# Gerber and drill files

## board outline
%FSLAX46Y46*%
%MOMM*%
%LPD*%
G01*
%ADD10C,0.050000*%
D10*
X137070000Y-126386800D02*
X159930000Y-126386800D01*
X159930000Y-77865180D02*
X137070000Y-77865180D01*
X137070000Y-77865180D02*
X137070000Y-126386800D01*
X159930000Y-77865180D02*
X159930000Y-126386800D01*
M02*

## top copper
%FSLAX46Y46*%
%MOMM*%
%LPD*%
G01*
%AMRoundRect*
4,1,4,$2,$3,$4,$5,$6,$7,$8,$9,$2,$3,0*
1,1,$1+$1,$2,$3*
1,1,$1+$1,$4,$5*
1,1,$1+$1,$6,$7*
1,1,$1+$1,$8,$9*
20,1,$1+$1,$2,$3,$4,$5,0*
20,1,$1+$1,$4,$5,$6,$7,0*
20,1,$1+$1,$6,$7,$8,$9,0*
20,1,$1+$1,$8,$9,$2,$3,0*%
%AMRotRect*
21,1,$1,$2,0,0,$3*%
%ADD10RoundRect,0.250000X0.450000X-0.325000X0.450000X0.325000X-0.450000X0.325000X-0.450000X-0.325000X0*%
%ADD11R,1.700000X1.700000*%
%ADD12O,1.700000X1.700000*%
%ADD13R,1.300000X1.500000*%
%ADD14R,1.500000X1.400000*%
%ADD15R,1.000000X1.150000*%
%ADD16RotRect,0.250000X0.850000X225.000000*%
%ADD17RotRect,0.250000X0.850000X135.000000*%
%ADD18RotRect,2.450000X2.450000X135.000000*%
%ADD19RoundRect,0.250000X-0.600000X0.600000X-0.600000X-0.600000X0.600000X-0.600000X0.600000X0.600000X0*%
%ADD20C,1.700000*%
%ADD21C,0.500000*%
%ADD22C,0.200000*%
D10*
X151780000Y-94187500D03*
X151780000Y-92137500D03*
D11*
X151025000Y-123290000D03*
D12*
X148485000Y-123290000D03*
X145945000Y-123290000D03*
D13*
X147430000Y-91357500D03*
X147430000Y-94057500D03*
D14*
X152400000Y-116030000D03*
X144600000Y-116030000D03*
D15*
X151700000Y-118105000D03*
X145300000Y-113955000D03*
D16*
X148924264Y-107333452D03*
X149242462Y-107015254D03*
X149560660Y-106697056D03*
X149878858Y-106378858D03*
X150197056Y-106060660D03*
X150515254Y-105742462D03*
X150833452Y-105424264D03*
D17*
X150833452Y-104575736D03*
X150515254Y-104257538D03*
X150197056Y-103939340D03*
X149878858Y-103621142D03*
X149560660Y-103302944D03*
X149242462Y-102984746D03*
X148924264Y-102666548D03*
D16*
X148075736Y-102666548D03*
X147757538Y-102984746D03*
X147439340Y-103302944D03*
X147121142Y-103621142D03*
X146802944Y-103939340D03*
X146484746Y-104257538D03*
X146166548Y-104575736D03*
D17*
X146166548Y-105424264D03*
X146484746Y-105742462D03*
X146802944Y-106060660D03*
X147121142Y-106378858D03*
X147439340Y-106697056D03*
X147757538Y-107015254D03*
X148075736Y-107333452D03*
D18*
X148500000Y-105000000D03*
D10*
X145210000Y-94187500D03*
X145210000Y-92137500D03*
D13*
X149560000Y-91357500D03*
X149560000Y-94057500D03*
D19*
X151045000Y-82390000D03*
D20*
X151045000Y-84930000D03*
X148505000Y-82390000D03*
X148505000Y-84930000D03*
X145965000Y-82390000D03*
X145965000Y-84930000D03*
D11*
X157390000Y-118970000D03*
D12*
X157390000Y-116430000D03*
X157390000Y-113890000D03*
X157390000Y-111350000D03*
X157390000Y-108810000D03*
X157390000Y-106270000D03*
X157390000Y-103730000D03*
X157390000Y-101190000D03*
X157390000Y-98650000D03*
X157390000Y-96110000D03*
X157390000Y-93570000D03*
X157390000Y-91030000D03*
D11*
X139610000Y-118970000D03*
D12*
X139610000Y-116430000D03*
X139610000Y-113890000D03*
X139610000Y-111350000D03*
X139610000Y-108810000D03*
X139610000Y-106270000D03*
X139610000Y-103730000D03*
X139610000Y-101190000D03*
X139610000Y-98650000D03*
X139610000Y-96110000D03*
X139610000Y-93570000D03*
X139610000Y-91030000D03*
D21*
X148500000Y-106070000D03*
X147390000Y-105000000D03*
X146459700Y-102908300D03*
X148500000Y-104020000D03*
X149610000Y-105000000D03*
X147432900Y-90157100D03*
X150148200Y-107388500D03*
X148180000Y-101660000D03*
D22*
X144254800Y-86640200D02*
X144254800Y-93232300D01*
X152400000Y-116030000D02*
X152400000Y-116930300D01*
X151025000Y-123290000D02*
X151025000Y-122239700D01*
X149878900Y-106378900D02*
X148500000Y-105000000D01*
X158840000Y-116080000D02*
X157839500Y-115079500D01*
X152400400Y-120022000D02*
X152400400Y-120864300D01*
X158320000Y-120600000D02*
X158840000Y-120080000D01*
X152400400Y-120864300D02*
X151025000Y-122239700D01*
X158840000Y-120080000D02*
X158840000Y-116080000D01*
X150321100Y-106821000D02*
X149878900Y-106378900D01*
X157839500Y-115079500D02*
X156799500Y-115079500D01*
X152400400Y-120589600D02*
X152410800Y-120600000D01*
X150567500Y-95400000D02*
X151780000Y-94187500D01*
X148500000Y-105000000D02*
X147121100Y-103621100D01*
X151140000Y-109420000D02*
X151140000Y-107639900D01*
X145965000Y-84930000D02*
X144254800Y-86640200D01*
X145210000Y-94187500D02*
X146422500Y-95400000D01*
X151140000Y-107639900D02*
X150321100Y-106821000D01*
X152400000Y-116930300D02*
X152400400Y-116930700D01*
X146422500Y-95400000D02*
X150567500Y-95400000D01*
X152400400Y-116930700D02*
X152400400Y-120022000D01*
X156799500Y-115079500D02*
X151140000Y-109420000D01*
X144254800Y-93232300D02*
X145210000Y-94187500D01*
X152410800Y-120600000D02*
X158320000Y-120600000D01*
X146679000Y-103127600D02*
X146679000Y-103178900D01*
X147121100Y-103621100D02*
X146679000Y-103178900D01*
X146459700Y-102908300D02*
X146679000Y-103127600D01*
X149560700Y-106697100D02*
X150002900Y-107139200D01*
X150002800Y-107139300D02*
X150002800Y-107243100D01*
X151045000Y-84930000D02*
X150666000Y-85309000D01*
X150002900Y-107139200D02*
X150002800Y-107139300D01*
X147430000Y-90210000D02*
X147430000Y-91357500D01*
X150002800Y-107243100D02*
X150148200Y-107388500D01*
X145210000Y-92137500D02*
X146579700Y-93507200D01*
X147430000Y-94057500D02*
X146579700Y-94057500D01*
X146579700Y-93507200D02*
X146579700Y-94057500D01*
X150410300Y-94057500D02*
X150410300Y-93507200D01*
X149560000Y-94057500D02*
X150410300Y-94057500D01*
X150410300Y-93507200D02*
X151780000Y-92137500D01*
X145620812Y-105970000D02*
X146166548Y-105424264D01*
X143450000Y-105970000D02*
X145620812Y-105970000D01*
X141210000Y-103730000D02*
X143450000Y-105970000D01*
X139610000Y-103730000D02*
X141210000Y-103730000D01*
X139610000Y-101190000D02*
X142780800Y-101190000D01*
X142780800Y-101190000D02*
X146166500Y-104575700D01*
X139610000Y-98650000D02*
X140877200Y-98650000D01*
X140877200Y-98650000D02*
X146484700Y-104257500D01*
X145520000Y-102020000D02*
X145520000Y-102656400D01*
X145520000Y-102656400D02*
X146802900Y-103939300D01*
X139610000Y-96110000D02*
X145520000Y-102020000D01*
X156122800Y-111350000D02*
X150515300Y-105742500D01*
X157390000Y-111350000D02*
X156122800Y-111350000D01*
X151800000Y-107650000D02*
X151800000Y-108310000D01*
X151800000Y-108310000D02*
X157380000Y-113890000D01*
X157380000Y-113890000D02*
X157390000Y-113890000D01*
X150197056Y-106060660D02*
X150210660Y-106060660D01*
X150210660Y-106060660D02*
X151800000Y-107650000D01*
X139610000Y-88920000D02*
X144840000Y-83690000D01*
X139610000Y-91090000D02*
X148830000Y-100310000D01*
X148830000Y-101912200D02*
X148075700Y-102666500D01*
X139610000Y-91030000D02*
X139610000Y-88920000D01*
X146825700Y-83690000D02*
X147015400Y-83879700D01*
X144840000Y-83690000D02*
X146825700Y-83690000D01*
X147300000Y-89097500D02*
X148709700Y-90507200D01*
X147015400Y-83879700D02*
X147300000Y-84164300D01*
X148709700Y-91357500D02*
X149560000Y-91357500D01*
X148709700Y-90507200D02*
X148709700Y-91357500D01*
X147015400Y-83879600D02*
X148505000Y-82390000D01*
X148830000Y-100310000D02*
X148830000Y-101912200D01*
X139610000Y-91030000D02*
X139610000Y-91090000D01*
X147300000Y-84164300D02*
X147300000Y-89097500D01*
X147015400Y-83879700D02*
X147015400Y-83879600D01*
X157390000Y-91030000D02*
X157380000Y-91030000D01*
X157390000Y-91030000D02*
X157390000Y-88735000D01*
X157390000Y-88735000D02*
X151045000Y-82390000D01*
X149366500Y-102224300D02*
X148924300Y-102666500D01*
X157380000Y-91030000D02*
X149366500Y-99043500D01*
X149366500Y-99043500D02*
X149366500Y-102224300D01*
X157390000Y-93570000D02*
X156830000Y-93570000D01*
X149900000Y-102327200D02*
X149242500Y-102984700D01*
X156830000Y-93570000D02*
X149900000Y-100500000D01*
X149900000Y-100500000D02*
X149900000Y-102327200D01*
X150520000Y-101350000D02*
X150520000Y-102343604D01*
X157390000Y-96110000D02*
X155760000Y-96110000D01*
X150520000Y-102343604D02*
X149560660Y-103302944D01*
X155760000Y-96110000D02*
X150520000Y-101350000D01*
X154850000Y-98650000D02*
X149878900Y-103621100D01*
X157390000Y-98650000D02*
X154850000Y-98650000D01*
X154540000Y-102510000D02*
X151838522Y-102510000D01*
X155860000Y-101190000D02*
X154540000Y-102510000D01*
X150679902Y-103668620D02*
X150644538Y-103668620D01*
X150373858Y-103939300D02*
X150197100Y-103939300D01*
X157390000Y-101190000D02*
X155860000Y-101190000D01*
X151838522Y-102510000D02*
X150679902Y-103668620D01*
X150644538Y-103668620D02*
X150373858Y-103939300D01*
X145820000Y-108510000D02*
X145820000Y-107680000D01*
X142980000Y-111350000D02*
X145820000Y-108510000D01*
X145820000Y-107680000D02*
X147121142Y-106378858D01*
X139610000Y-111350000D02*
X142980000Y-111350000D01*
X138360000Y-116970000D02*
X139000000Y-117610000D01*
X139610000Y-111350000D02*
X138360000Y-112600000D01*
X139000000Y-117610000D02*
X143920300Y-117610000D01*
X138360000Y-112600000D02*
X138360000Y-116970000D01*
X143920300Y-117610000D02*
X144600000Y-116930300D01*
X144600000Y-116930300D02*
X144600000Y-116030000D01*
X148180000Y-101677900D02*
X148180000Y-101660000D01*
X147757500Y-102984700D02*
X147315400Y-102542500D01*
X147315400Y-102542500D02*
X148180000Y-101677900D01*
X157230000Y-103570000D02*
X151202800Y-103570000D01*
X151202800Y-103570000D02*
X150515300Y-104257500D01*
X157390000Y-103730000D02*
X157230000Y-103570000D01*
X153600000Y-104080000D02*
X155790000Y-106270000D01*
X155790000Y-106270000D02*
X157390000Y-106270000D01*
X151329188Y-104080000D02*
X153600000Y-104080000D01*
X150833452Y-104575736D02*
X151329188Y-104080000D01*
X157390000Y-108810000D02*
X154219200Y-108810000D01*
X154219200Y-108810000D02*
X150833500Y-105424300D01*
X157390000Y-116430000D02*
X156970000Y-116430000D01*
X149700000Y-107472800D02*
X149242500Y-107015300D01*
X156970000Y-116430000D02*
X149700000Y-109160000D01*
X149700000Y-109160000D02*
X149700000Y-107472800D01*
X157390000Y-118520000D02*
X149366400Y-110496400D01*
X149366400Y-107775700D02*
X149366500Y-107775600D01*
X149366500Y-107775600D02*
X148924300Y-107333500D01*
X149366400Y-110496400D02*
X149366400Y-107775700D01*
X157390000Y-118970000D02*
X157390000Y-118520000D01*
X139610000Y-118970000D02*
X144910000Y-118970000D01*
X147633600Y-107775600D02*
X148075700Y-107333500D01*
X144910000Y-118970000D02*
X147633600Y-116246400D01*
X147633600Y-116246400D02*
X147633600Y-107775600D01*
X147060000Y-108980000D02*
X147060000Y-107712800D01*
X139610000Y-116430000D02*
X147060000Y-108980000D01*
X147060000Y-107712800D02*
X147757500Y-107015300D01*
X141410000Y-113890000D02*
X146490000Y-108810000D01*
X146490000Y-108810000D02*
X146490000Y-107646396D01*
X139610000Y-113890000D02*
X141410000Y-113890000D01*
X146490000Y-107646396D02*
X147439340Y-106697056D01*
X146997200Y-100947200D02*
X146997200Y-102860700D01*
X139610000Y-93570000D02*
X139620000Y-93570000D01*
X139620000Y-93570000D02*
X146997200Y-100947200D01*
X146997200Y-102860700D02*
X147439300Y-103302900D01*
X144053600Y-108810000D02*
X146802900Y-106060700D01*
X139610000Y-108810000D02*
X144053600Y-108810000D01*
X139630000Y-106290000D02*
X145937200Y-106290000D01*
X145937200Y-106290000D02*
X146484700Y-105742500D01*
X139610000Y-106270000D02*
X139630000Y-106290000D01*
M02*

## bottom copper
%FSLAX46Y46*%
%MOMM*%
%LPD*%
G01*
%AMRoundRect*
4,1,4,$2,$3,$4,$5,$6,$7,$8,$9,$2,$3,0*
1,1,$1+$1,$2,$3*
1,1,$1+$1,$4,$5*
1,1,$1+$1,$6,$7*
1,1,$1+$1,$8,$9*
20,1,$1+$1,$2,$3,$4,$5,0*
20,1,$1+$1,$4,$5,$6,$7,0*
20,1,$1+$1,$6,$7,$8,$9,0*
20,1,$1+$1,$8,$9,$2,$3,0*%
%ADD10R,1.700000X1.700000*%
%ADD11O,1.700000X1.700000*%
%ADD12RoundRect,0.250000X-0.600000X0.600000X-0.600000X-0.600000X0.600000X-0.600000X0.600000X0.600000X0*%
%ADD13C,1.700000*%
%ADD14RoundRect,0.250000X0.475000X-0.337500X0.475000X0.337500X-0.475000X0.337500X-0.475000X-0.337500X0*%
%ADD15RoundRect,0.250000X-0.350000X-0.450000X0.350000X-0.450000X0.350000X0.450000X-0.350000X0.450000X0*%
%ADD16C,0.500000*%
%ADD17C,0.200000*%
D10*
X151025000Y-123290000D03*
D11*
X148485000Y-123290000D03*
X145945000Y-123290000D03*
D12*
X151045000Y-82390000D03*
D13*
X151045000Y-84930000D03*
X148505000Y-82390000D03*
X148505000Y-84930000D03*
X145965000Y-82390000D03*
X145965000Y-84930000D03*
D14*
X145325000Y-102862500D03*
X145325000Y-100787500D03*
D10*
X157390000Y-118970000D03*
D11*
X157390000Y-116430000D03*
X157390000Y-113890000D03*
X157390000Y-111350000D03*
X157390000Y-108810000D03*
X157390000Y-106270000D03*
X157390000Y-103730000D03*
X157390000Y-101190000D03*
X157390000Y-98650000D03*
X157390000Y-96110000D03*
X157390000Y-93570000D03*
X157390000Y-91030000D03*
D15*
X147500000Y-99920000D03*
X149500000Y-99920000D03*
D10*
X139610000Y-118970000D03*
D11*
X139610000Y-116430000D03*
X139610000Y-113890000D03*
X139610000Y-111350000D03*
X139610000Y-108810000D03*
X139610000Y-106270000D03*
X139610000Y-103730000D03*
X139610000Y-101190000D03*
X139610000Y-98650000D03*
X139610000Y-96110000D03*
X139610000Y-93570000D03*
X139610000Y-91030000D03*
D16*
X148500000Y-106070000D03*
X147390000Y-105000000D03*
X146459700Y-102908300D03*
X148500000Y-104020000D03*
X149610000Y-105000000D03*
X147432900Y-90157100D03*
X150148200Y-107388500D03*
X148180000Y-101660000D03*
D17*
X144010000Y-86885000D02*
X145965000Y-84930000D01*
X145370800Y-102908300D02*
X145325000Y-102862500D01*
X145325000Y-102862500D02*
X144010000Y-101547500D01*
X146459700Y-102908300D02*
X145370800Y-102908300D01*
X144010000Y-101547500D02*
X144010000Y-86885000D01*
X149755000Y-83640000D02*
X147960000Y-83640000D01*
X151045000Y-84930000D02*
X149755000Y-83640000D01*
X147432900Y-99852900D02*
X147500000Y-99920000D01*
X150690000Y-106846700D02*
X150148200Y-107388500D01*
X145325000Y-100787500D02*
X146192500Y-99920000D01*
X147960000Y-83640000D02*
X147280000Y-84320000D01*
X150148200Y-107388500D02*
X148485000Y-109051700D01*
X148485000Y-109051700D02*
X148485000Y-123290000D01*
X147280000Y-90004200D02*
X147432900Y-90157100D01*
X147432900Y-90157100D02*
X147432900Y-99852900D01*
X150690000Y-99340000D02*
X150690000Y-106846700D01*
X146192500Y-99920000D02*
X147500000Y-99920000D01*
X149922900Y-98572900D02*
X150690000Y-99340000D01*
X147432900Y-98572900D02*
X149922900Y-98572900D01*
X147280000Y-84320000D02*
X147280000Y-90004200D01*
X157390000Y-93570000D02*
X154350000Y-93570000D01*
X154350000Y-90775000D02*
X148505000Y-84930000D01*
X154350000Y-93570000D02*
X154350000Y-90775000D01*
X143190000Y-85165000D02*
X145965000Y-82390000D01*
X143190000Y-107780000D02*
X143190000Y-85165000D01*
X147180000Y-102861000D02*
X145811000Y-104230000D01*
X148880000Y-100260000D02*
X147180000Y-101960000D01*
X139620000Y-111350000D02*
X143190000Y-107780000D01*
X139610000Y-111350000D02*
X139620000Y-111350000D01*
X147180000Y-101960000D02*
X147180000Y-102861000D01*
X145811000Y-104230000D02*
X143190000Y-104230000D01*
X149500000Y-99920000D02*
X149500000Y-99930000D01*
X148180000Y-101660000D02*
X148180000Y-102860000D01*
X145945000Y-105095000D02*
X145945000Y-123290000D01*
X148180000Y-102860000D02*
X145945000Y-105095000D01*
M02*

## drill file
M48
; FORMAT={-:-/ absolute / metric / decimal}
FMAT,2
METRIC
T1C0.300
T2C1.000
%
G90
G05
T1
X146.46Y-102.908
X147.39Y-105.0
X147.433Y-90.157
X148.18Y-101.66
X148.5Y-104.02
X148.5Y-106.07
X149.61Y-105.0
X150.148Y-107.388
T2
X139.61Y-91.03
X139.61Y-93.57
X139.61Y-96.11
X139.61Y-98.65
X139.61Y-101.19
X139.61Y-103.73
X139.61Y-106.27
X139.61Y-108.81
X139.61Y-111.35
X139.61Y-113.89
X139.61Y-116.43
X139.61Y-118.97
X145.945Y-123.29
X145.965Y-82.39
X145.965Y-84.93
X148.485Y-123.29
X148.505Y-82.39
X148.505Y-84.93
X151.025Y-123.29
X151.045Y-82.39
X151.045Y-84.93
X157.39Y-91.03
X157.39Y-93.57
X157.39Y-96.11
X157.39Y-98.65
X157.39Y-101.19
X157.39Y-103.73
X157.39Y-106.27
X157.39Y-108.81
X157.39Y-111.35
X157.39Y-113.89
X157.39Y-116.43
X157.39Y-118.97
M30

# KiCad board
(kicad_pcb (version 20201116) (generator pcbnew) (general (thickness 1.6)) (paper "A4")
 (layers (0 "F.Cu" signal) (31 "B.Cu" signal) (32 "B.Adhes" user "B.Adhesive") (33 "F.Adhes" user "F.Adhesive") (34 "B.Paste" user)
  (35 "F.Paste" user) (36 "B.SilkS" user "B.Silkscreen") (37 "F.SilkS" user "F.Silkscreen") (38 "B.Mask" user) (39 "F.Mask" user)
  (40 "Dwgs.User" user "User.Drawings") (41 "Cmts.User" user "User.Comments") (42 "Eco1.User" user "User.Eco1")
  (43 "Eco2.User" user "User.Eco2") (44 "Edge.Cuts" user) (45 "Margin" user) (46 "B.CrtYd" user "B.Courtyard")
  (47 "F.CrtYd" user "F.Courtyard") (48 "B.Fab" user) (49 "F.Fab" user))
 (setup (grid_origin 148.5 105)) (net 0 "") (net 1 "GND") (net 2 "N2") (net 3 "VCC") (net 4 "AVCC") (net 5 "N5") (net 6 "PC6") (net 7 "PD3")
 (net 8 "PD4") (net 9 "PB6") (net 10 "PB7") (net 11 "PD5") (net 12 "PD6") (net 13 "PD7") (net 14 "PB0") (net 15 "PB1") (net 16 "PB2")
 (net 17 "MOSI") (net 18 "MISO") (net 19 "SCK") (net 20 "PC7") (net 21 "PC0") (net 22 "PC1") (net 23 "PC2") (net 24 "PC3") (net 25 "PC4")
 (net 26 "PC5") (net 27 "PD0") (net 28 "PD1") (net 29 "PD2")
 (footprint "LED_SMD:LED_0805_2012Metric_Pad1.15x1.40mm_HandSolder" (layer "F.Cu") (at 151.78 93.1625 90)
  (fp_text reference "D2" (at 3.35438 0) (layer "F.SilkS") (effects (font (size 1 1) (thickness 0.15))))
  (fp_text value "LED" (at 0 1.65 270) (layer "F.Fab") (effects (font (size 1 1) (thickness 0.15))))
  (pad "1" smd roundrect (at -1.025 0 90) (size 1.15 1.4) (layers "F.Cu" "F.Paste" "F.Mask") (roundrect_rratio 0.217391) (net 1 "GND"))
  (pad "2" smd roundrect (at 1.025 0 90) (size 1.15 1.4) (layers "F.Cu" "F.Paste" "F.Mask") (roundrect_rratio 0.217391) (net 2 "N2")))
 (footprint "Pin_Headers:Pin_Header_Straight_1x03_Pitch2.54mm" (layer "F.Cu") (at 151.025 123.29 -90)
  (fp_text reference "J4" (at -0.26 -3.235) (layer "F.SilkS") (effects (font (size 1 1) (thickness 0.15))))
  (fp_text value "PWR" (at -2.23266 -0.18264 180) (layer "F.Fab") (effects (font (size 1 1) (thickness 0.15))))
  (pad "1" thru_hole rect (at 0 0 270) (size 1.7 1.7) (drill 1) (layers *.Cu *.Mask) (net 1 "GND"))
  (pad "2" thru_hole oval (at 0 2.54 270) (size 1.7 1.7) (drill 1) (layers *.Cu *.Mask) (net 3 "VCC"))
  (pad "3" thru_hole oval (at 0 5.08 270) (size 1.7 1.7) (drill 1) (layers *.Cu *.Mask) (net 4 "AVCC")))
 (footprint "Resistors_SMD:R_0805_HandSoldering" (layer "F.Cu") (at 147.43 92.7075 -90)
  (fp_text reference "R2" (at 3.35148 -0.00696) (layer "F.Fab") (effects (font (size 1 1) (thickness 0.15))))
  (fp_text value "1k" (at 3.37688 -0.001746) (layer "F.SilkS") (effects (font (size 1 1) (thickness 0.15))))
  (pad "1" smd rect (at -1.35 0 270) (size 1.5 1.3) (layers "F.Cu" "F.Paste" "F.Mask") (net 3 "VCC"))
  (pad "2" smd rect (at 1.35 0 270) (size 1.5 1.3) (layers "F.Cu" "F.Paste" "F.Mask") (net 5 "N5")))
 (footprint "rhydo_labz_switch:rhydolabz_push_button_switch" (layer "F.Cu") (at 148.5 116.03 180)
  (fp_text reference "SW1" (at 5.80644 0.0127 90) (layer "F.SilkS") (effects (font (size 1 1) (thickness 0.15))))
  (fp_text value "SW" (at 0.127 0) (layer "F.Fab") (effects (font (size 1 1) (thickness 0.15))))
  (pad "1" smd rect (at -3.9 0 180) (size 1.5 1.4) (layers "F.Cu" "F.Paste" "F.Mask") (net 1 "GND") (solder_mask_margin 0.000254))
  (pad "2" smd rect (at 3.9 0 180) (size 1.5 1.4) (layers "F.Cu" "F.Paste" "F.Mask") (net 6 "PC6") (solder_mask_margin 0.000254))
  (pad "3" smd rect (at -3.2 -2.075 180) (size 1 1.15) (layers "F.Cu" "F.Paste" "F.Mask") (solder_mask_margin 0.000254))
  (pad "4" smd rect (at 3.2 2.075 180) (size 1 1.15) (layers "F.Cu" "F.Paste" "F.Mask") (solder_mask_margin 0.000254)))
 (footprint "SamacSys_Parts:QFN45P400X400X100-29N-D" (layer "F.Cu") (at 148.5 105 135)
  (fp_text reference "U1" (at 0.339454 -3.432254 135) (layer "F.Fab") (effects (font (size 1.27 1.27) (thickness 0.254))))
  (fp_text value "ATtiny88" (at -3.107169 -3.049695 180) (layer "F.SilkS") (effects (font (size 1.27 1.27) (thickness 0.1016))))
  (pad "1" smd rect (at -1.95 -1.35 225) (size 0.25 0.85) (layers "F.Cu" "F.Paste" "F.Mask") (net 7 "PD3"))
  (pad "2" smd rect (at -1.95 -0.9 225) (size 0.25 0.85) (layers "F.Cu" "F.Paste" "F.Mask") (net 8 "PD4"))
  (pad "3" smd rect (at -1.95 -0.45 225) (size 0.25 0.85) (layers "F.Cu" "F.Paste" "F.Mask") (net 3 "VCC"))
  (pad "4" smd rect (at -1.95 0 225) (size 0.25 0.85) (layers "F.Cu" "F.Paste" "F.Mask") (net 1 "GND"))
  (pad "5" smd rect (at -1.95 0.45 225) (size 0.25 0.85) (layers "F.Cu" "F.Paste" "F.Mask") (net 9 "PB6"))
  (pad "6" smd rect (at -1.95 0.9 225) (size 0.25 0.85) (layers "F.Cu" "F.Paste" "F.Mask") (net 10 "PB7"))
  (pad "7" smd rect (at -1.95 1.35 225) (size 0.25 0.85) (layers "F.Cu" "F.Paste" "F.Mask") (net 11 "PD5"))
  (pad "8" smd rect (at -1.35 1.95 135) (size 0.25 0.85) (layers "F.Cu" "F.Paste" "F.Mask") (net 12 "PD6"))
  (pad "9" smd rect (at -0.9 1.95 135) (size 0.25 0.85) (layers "F.Cu" "F.Paste" "F.Mask") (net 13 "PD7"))
  (pad "10" smd rect (at -0.45 1.95 135) (size 0.25 0.85) (layers "F.Cu" "F.Paste" "F.Mask") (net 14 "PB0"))
  (pad "11" smd rect (at 0 1.95 135) (size 0.25 0.85) (layers "F.Cu" "F.Paste" "F.Mask") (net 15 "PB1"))
  (pad "12" smd rect (at 0.45 1.95 135) (size 0.25 0.85) (layers "F.Cu" "F.Paste" "F.Mask") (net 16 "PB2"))
  (pad "13" smd rect (at 0.9 1.95 135) (size 0.25 0.85) (layers "F.Cu" "F.Paste" "F.Mask") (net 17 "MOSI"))
  (pad "14" smd rect (at 1.35 1.95 135) (size 0.25 0.85) (layers "F.Cu" "F.Paste" "F.Mask") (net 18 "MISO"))
  (pad "15" smd rect (at 1.95 1.35 225) (size 0.25 0.85) (layers "F.Cu" "F.Paste" "F.Mask") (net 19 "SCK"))
  (pad "16" smd rect (at 1.95 0.9 225) (size 0.25 0.85) (layers "F.Cu" "F.Paste" "F.Mask") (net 4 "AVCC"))
  (pad "17" smd rect (at 1.95 0.45 225) (size 0.25 0.85) (layers "F.Cu" "F.Paste" "F.Mask") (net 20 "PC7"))
  (pad "18" smd rect (at 1.95 0 225) (size 0.25 0.85) (layers "F.Cu" "F.Paste" "F.Mask") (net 1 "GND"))
  (pad "19" smd rect (at 1.95 -0.45 225) (size 0.25 0.85) (layers "F.Cu" "F.Paste" "F.Mask") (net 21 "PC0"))
  (pad "20" smd rect (at 1.95 -0.9 225) (size 0.25 0.85) (layers "F.Cu" "F.Paste" "F.Mask") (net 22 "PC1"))
  (pad "21" smd rect (at 1.95 -1.35 225) (size 0.25 0.85) (layers "F.Cu" "F.Paste" "F.Mask") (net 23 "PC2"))
  (pad "22" smd rect (at 1.35 -1.95 135) (size 0.25 0.85) (layers "F.Cu" "F.Paste" "F.Mask") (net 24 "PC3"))
  (pad "23" smd rect (at 0.9 -1.95 135) (size 0.25 0.85) (layers "F.Cu" "F.Paste" "F.Mask") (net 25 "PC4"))
  (pad "24" smd rect (at 0.45 -1.95 135) (size 0.25 0.85) (layers "F.Cu" "F.Paste" "F.Mask") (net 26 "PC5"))
  (pad "25" smd rect (at 0 -1.95 135) (size 0.25 0.85) (layers "F.Cu" "F.Paste" "F.Mask") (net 6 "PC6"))
  (pad "26" smd rect (at -0.45 -1.95 135) (size 0.25 0.85) (layers "F.Cu" "F.Paste" "F.Mask") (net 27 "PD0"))
  (pad "27" smd rect (at -0.9 -1.95 135) (size 0.25 0.85) (layers "F.Cu" "F.Paste" "F.Mask") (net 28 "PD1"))
  (pad "28" smd rect (at -1.35 -1.95 135) (size 0.25 0.85) (layers "F.Cu" "F.Paste" "F.Mask") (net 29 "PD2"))
  (pad "29" smd rect (at 0 0 135) (size 2.45 2.45) (layers "F.Cu" "F.Paste" "F.Mask") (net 1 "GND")))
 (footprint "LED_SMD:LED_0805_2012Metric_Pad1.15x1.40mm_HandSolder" (layer "F.Cu") (at 145.21 93.1625 90)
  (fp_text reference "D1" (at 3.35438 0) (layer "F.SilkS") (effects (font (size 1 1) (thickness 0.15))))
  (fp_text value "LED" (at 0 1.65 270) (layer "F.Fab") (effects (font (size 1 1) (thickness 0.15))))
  (pad "1" smd roundrect (at -1.025 0 90) (size 1.15 1.4) (layers "F.Cu" "F.Paste" "F.Mask") (roundrect_rratio 0.217391) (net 1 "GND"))
  (pad "2" smd roundrect (at 1.025 0 90) (size 1.15 1.4) (layers "F.Cu" "F.Paste" "F.Mask") (roundrect_rratio 0.217391) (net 5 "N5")))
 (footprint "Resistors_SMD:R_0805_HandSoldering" (layer "F.Cu") (at 149.56 92.7075 -90)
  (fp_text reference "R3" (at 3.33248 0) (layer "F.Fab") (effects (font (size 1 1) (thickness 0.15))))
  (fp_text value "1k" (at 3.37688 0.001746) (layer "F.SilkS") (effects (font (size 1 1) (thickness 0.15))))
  (pad "1" smd rect (at -1.35 0 270) (size 1.5 1.3) (layers "F.Cu" "F.Paste" "F.Mask") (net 19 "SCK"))
  (pad "2" smd rect (at 1.35 0 270) (size 1.5 1.3) (layers "F.Cu" "F.Paste" "F.Mask") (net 2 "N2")))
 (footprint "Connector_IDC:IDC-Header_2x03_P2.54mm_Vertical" (layer "F.Cu") (at 151.045 82.39 -90)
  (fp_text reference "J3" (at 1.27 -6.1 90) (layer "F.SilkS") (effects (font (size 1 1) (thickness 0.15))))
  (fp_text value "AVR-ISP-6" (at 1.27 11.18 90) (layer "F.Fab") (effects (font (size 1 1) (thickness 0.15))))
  (pad "1" thru_hole roundrect (at 0 0 270) (size 1.7 1.7) (drill 1) (layers *.Cu *.Mask) (roundrect_rratio 0.147059) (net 18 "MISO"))
  (pad "2" thru_hole circle (at 2.54 0 270) (size 1.7 1.7) (drill 1) (layers *.Cu *.Mask) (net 3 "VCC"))
  (pad "3" thru_hole circle (at 0 2.54 270) (size 1.7 1.7) (drill 1) (layers *.Cu *.Mask) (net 19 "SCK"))
  (pad "4" thru_hole circle (at 2.54 2.54 270) (size 1.7 1.7) (drill 1) (layers *.Cu *.Mask) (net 17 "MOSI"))
  (pad "5" thru_hole circle (at 0 5.08 270) (size 1.7 1.7) (drill 1) (layers *.Cu *.Mask) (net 6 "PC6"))
  (pad "6" thru_hole circle (at 2.54 5.08 270) (size 1.7 1.7) (drill 1) (layers *.Cu *.Mask) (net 1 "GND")))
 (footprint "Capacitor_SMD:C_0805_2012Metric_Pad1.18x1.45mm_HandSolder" (layer "B.Cu") (at 145.325 101.825 90)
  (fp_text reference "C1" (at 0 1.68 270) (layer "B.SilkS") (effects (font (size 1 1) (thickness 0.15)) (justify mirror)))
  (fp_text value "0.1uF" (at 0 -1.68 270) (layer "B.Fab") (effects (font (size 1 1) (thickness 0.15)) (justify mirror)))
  (pad "1" smd roundrect (at -1.0375 0 90) (size 1.175 1.45) (layers "B.Cu" "B.Paste" "B.Mask") (roundrect_rratio 0.212766) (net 1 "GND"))
  (pad "2" smd roundrect (at 1.0375 0 90) (size 1.175 1.45) (layers "B.Cu" "B.Paste" "B.Mask") (roundrect_rratio 0.212766) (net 3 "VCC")))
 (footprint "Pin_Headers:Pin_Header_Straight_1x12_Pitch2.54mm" (layer "B.Cu") (at 157.39 118.97)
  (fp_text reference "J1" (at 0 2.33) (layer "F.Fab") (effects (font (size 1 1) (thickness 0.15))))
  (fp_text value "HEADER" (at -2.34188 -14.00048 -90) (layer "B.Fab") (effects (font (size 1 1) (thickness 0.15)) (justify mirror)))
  (pad "1" thru_hole rect (at 0 0) (size 1.7 1.7) (drill 1) (layers *.Cu *.Mask) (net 7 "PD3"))
  (pad "2" thru_hole oval (at 0 -2.54) (size 1.7 1.7) (drill 1) (layers *.Cu *.Mask) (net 8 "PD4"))
  (pad "3" thru_hole oval (at 0 -5.08) (size 1.7 1.7) (drill 1) (layers *.Cu *.Mask) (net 9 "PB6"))
  (pad "4" thru_hole oval (at 0 -7.62) (size 1.7 1.7) (drill 1) (layers *.Cu *.Mask) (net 10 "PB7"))
  (pad "5" thru_hole oval (at 0 -10.16) (size 1.7 1.7) (drill 1) (layers *.Cu *.Mask) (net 11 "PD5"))
  (pad "6" thru_hole oval (at 0 -12.7) (size 1.7 1.7) (drill 1) (layers *.Cu *.Mask) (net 12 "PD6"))
  (pad "7" thru_hole oval (at 0 -15.24) (size 1.7 1.7) (drill 1) (layers *.Cu *.Mask) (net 13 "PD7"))
  (pad "8" thru_hole oval (at 0 -17.78) (size 1.7 1.7) (drill 1) (layers *.Cu *.Mask) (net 14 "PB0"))
  (pad "9" thru_hole oval (at 0 -20.32) (size 1.7 1.7) (drill 1) (layers *.Cu *.Mask) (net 15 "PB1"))
  (pad "10" thru_hole oval (at 0 -22.86) (size 1.7 1.7) (drill 1) (layers *.Cu *.Mask) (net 16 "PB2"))
  (pad "11" thru_hole oval (at 0 -25.4) (size 1.7 1.7) (drill 1) (layers *.Cu *.Mask) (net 17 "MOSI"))
  (pad "12" thru_hole oval (at 0 -27.94) (size 1.7 1.7) (drill 1) (layers *.Cu *.Mask) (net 18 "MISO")))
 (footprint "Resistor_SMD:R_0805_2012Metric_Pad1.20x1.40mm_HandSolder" (layer "B.Cu") (at 148.5 99.92)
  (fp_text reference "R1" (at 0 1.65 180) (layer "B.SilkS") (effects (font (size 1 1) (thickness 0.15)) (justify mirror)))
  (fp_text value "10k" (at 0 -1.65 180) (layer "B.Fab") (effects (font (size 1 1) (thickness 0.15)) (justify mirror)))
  (pad "1" smd roundrect (at -1 0) (size 1.2 1.4) (layers "B.Cu" "B.Paste" "B.Mask") (roundrect_rratio 0.208333) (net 3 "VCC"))
  (pad "2" smd roundrect (at 1 0) (size 1.2 1.4) (layers "B.Cu" "B.Paste" "B.Mask") (roundrect_rratio 0.208333) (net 6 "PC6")))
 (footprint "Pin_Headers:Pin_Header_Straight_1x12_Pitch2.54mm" (layer "B.Cu") (at 139.61 118.97)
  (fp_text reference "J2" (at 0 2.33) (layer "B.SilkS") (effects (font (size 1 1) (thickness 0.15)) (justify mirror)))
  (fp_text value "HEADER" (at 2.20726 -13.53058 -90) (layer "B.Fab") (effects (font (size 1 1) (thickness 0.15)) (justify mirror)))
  (pad "1" thru_hole rect (at 0 0) (size 1.7 1.7) (drill 1) (layers *.Cu *.Mask) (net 29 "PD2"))
  (pad "2" thru_hole oval (at 0 -2.54) (size 1.7 1.7) (drill 1) (layers *.Cu *.Mask) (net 28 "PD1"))
  (pad "3" thru_hole oval (at 0 -5.08) (size 1.7 1.7) (drill 1) (layers *.Cu *.Mask) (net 27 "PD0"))
  (pad "4" thru_hole oval (at 0 -7.62) (size 1.7 1.7) (drill 1) (layers *.Cu *.Mask) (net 6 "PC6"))
  (pad "5" thru_hole oval (at 0 -10.16) (size 1.7 1.7) (drill 1) (layers *.Cu *.Mask) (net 26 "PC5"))
  (pad "6" thru_hole oval (at 0 -12.7) (size 1.7 1.7) (drill 1) (layers *.Cu *.Mask) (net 25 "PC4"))
  (pad "7" thru_hole oval (at 0 -15.24) (size 1.7 1.7) (drill 1) (layers *.Cu *.Mask) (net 24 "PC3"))
  (pad "8" thru_hole oval (at 0 -17.78) (size 1.7 1.7) (drill 1) (layers *.Cu *.Mask) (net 23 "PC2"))
  (pad "9" thru_hole oval (at 0 -20.32) (size 1.7 1.7) (drill 1) (layers *.Cu *.Mask) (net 22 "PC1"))
  (pad "10" thru_hole oval (at 0 -22.86) (size 1.7 1.7) (drill 1) (layers *.Cu *.Mask) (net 21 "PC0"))
  (pad "11" thru_hole oval (at 0 -25.4) (size 1.7 1.7) (drill 1) (layers *.Cu *.Mask) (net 20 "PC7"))
  (pad "12" thru_hole oval (at 0 -27.94) (size 1.7 1.7) (drill 1) (layers *.Cu *.Mask) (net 19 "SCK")))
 (gr_line (start 137.07 126.3868) (end 159.93 126.3868) (layer "Edge.Cuts") (width 0.05))
 (gr_line (start 159.93 77.86518) (end 137.07 77.86518) (layer "Edge.Cuts") (width 0.05))
 (gr_line (start 137.07 77.86518) (end 137.07 126.3868) (layer "Edge.Cuts") (width 0.05))
 (gr_line (start 159.93 77.86518) (end 159.93 126.3868) (layer "Edge.Cuts") (width 0.05))
 (segment (start 144.2548 86.6402) (end 144.2548 93.2323) (width 0.2) (layer "F.Cu") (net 1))
 (segment (start 152.4 116.03) (end 152.4 116.9303) (width 0.2) (layer "F.Cu") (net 1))
 (segment (start 151.025 123.29) (end 151.025 122.2397) (width 0.2) (layer "F.Cu") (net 1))
 (segment (start 149.8789 106.3789) (end 148.5 105) (width 0.2) (layer "F.Cu") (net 1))
 (segment (start 158.84 116.08) (end 157.8395 115.0795) (width 0.2) (layer "F.Cu") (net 1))
 (segment (start 152.4004 120.022) (end 152.4004 120.8643) (width 0.2) (layer "F.Cu") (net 1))
 (segment (start 158.32 120.6) (end 158.84 120.08) (width 0.2) (layer "F.Cu") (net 1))
 (segment (start 152.4004 120.8643) (end 151.025 122.2397) (width 0.2) (layer "F.Cu") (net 1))
 (segment (start 158.84 120.08) (end 158.84 116.08) (width 0.2) (layer "F.Cu") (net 1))
 (segment (start 150.3211 106.821) (end 149.8789 106.3789) (width 0.2) (layer "F.Cu") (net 1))
 (segment (start 157.8395 115.0795) (end 156.7995 115.0795) (width 0.2) (layer "F.Cu") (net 1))
 (segment (start 152.4004 120.5896) (end 152.4108 120.6) (width 0.2) (layer "F.Cu") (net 1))
 (segment (start 150.5675 95.4) (end 151.78 94.1875) (width 0.2) (layer "F.Cu") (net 1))
 (segment (start 148.5 105) (end 147.1211 103.6211) (width 0.2) (layer "F.Cu") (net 1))
 (segment (start 151.14 109.42) (end 151.14 107.6399) (width 0.2) (layer "F.Cu") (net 1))
 (segment (start 145.965 84.93) (end 144.2548 86.6402) (width 0.2) (layer "F.Cu") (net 1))
 (segment (start 145.21 94.1875) (end 146.4225 95.4) (width 0.2) (layer "F.Cu") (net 1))
 (segment (start 151.14 107.6399) (end 150.3211 106.821) (width 0.2) (layer "F.Cu") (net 1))
 (segment (start 152.4 116.9303) (end 152.4004 116.9307) (width 0.2) (layer "F.Cu") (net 1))
 (segment (start 146.4225 95.4) (end 150.5675 95.4) (width 0.2) (layer "F.Cu") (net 1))
 (segment (start 152.4004 116.9307) (end 152.4004 120.022) (width 0.2) (layer "F.Cu") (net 1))
 (segment (start 156.7995 115.0795) (end 151.14 109.42) (width 0.2) (layer "F.Cu") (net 1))
 (segment (start 144.2548 93.2323) (end 145.21 94.1875) (width 0.2) (layer "F.Cu") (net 1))
 (segment (start 152.4108 120.6) (end 158.32 120.6) (width 0.2) (layer "F.Cu") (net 1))
 (segment (start 146.679 103.1276) (end 146.679 103.1789) (width 0.2) (layer "F.Cu") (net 1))
 (segment (start 147.1211 103.6211) (end 146.679 103.1789) (width 0.2) (layer "F.Cu") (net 1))
 (segment (start 146.4597 102.9083) (end 146.679 103.1276) (width 0.2) (layer "F.Cu") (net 1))
 (via (at 148.5 106.07) (size 0.5) (drill 0.3) (layers "F.Cu" "B.Cu") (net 1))
 (via (at 147.39 105) (size 0.5) (drill 0.3) (layers "F.Cu" "B.Cu") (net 1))
 (via (at 146.4597 102.9083) (size 0.5) (layers "F.Cu" "B.Cu") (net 1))
 (via (at 148.5 104.02) (size 0.5) (drill 0.3) (layers "F.Cu" "B.Cu") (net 1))
 (via (at 149.61 105) (size 0.5) (drill 0.3) (layers "F.Cu" "B.Cu") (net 1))
 (segment (start 144.01 86.885) (end 145.965 84.93) (width 0.2) (layer "B.Cu") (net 1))
 (segment (start 145.3708 102.9083) (end 145.325 102.8625) (width 0.2) (layer "B.Cu") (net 1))
 (segment (start 145.325 102.8625) (end 144.01 101.5475) (width 0.2) (layer "B.Cu") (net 1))
 (segment (start 146.4597 102.9083) (end 145.3708 102.9083) (width 0.2) (layer "B.Cu") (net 1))
 (segment (start 144.01 101.5475) (end 144.01 86.885) (width 0.2) (layer "B.Cu") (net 1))
 (segment (start 149.5607 106.6971) (end 150.0029 107.1392) (width 0.2) (layer "F.Cu") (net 3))
 (segment (start 150.0028 107.1393) (end 150.0028 107.2431) (width 0.2) (layer "F.Cu") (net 3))
 (segment (start 151.045 84.93) (end 150.666 85.309) (width 0.2) (layer "F.Cu") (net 3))
 (segment (start 150.0029 107.1392) (end 150.0028 107.1393) (width 0.2) (layer "F.Cu") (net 3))
 (segment (start 147.43 90.21) (end 147.43 91.3575) (width 0.2) (layer "F.Cu") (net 3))
 (segment (start 150.0028 107.2431) (end 150.1482 107.3885) (width 0.2) (layer "F.Cu") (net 3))
 (via (at 147.4329 90.1571) (size 0.5) (drill 0.3) (layers "F.Cu" "B.Cu") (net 3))
 (via (at 150.1482 107.3885) (size 0.5) (layers "F.Cu" "B.Cu") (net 3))
 (segment (start 149.755 83.64) (end 147.96 83.64) (width 0.2) (layer "B.Cu") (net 3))
 (segment (start 151.045 84.93) (end 149.755 83.64) (width 0.2) (layer "B.Cu") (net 3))
 (segment (start 147.4329 99.8529) (end 147.5 99.92) (width 0.2) (layer "B.Cu") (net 3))
 (segment (start 150.69 106.8467) (end 150.1482 107.3885) (width 0.2) (layer "B.Cu") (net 3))
 (segment (start 145.325 100.7875) (end 146.1925 99.92) (width 0.2) (layer "B.Cu") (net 3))
 (segment (start 147.96 83.64) (end 147.28 84.32) (width 0.2) (layer "B.Cu") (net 3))
 (segment (start 150.1482 107.3885) (end 148.485 109.0517) (width 0.2) (layer "B.Cu") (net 3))
 (segment (start 148.485 109.0517) (end 148.485 123.29) (width 0.2) (layer "B.Cu") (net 3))
 (segment (start 147.28 90.0042) (end 147.4329 90.1571) (width 0.2) (layer "B.Cu") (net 3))
 (segment (start 147.4329 90.1571) (end 147.4329 99.8529) (width 0.2) (layer "B.Cu") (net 3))
 (segment (start 150.69 99.34) (end 150.69 106.8467) (width 0.2) (layer "B.Cu") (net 3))
 (segment (start 146.1925 99.92) (end 147.5 99.92) (width 0.2) (layer "B.Cu") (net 3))
 (segment (start 149.9229 98.5729) (end 150.69 99.34) (width 0.2) (layer "B.Cu") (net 3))
 (segment (start 147.4329 98.5729) (end 149.9229 98.5729) (width 0.2) (layer "B.Cu") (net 3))
 (segment (start 147.28 84.32) (end 147.28 90.0042) (width 0.2) (layer "B.Cu") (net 3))
 (segment (start 145.21 92.1375) (end 146.5797 93.5072) (width 0.2) (layer "F.Cu") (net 5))
 (segment (start 147.43 94.0575) (end 146.5797 94.0575) (width 0.2) (layer "F.Cu") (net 5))
 (segment (start 146.5797 93.5072) (end 146.5797 94.0575) (width 0.2) (layer "F.Cu") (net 5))
 (segment (start 150.4103 94.0575) (end 150.4103 93.5072) (width 0.2) (layer "F.Cu") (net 2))
 (segment (start 149.56 94.0575) (end 150.4103 94.0575) (width 0.2) (layer "F.Cu") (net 2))
 (segment (start 150.4103 93.5072) (end 151.78 92.1375) (width 0.2) (layer "F.Cu") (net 2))
 (segment (start 145.620812 105.97) (end 146.166548 105.424264) (width 0.2) (layer "F.Cu") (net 24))
 (segment (start 143.45 105.97) (end 145.620812 105.97) (width 0.2) (layer "F.Cu") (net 24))
 (segment (start 141.21 103.73) (end 143.45 105.97) (width 0.2) (layer "F.Cu") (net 24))
 (segment (start 139.61 103.73) (end 141.21 103.73) (width 0.2) (layer "F.Cu") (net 24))
 (segment (start 139.61 101.19) (end 142.7808 101.19) (width 0.2) (layer "F.Cu") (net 23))
 (segment (start 142.7808 101.19) (end 146.1665 104.5757) (width 0.2) (layer "F.Cu") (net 23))
 (segment (start 139.61 98.65) (end 140.8772 98.65) (width 0.2) (layer "F.Cu") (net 22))
 (segment (start 140.8772 98.65) (end 146.4847 104.2575) (width 0.2) (layer "F.Cu") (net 22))
 (segment (start 145.52 102.02) (end 145.52 102.6564) (width 0.2) (layer "F.Cu") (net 21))
 (segment (start 145.52 102.6564) (end 146.8029 103.9393) (width 0.2) (layer "F.Cu") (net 21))
 (segment (start 139.61 96.11) (end 145.52 102.02) (width 0.2) (layer "F.Cu") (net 21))
 (segment (start 156.1228 111.35) (end 150.5153 105.7425) (width 0.2) (layer "F.Cu") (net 10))
 (segment (start 157.39 111.35) (end 156.1228 111.35) (width 0.2) (layer "F.Cu") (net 10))
 (segment (start 151.8 107.65) (end 151.8 108.31) (width 0.2) (layer "F.Cu") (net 9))
 (segment (start 151.8 108.31) (end 157.38 113.89) (width 0.2) (layer "F.Cu") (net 9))
 (segment (start 157.38 113.89) (end 157.39 113.89) (width 0.2) (layer "F.Cu") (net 9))
 (segment (start 150.197056 106.06066) (end 150.21066 106.06066) (width 0.2) (layer "F.Cu") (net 9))
 (segment (start 150.21066 106.06066) (end 151.8 107.65) (width 0.2) (layer "F.Cu") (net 9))
 (segment (start 139.61 88.92) (end 144.84 83.69) (width 0.2) (layer "F.Cu") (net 19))
 (segment (start 139.61 91.09) (end 148.83 100.31) (width 0.2) (layer "F.Cu") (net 19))
 (segment (start 148.83 101.9122) (end 148.0757 102.6665) (width 0.2) (layer "F.Cu") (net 19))
 (segment (start 139.61 91.03) (end 139.61 88.92) (width 0.2) (layer "F.Cu") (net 19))
 (segment (start 146.8257 83.69) (end 147.0154 83.8797) (width 0.2) (layer "F.Cu") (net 19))
 (segment (start 144.84 83.69) (end 146.8257 83.69) (width 0.2) (layer "F.Cu") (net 19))
 (segment (start 147.3 89.0975) (end 148.7097 90.5072) (width 0.2) (layer "F.Cu") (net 19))
 (segment (start 147.0154 83.8797) (end 147.3 84.1643) (width 0.2) (layer "F.Cu") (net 19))
 (segment (start 148.7097 91.3575) (end 149.56 91.3575) (width 0.2) (layer "F.Cu") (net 19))
 (segment (start 148.7097 90.5072) (end 148.7097 91.3575) (width 0.2) (layer "F.Cu") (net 19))
 (segment (start 147.0154 83.8796) (end 148.505 82.39) (width 0.2) (layer "F.Cu") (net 19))
 (segment (start 148.83 100.31) (end 148.83 101.9122) (width 0.2) (layer "F.Cu") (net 19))
 (segment (start 139.61 91.03) (end 139.61 91.09) (width 0.2) (layer "F.Cu") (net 19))
 (segment (start 147.3 84.1643) (end 147.3 89.0975) (width 0.2) (layer "F.Cu") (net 19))
 (segment (start 147.0154 83.8797) (end 147.0154 83.8796) (width 0.2) (layer "F.Cu") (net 19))
 (segment (start 157.39 91.03) (end 157.38 91.03) (width 0.2) (layer "F.Cu") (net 18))
 (segment (start 157.39 91.03) (end 157.39 88.735) (width 0.2) (layer "F.Cu") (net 18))
 (segment (start 157.39 88.735) (end 151.045 82.39) (width 0.2) (layer "F.Cu") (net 18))
 (segment (start 149.3665 102.2243) (end 148.9243 102.6665) (width 0.2) (layer "F.Cu") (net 18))
 (segment (start 157.38 91.03) (end 149.3665 99.0435) (width 0.2) (layer "F.Cu") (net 18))
 (segment (start 149.3665 99.0435) (end 149.3665 102.2243) (width 0.2) (layer "F.Cu") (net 18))
 (segment (start 157.39 93.57) (end 156.83 93.57) (width 0.2) (layer "F.Cu") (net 17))
 (segment (start 149.9 102.3272) (end 149.2425 102.9847) (width 0.2) (layer "F.Cu") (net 17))
 (segment (start 156.83 93.57) (end 149.9 100.5) (width 0.2) (layer "F.Cu") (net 17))
 (segment (start 149.9 100.5) (end 149.9 102.3272) (width 0.2) (layer "F.Cu") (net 17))
 (segment (start 157.39 93.57) (end 154.35 93.57) (width 0.2) (layer "B.Cu") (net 17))
 (segment (start 154.35 90.775) (end 148.505 84.93) (width 0.2) (layer "B.Cu") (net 17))
 (segment (start 154.35 93.57) (end 154.35 90.775) (width 0.2) (layer "B.Cu") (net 17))
 (segment (start 150.52 101.35) (end 150.52 102.343604) (width 0.2) (layer "F.Cu") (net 16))
 (segment (start 157.39 96.11) (end 155.76 96.11) (width 0.2) (layer "F.Cu") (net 16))
 (segment (start 150.52 102.343604) (end 149.56066 103.302944) (width 0.2) (layer "F.Cu") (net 16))
 (segment (start 155.76 96.11) (end 150.52 101.35) (width 0.2) (layer "F.Cu") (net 16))
 (segment (start 154.85 98.65) (end 149.8789 103.6211) (width 0.2) (layer "F.Cu") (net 15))
 (segment (start 157.39 98.65) (end 154.85 98.65) (width 0.2) (layer "F.Cu") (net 15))
 (segment (start 154.54 102.51) (end 151.838522 102.51) (width 0.2) (layer "F.Cu") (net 14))
 (segment (start 155.86 101.19) (end 154.54 102.51) (width 0.2) (layer "F.Cu") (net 14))
 (segment (start 150.679902 103.66862) (end 150.644538 103.66862) (width 0.2) (layer "F.Cu") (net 14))
 (segment (start 150.373858 103.9393) (end 150.1971 103.9393) (width 0.2) (layer "F.Cu") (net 14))
 (segment (start 157.39 101.19) (end 155.86 101.19) (width 0.2) (layer "F.Cu") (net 14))
 (segment (start 151.838522 102.51) (end 150.679902 103.66862) (width 0.2) (layer "F.Cu") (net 14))
 (segment (start 150.644538 103.66862) (end 150.373858 103.9393) (width 0.2) (layer "F.Cu") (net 14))
 (segment (start 145.82 108.51) (end 145.82 107.68) (width 0.2) (layer "F.Cu") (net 6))
 (segment (start 142.98 111.35) (end 145.82 108.51) (width 0.2) (layer "F.Cu") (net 6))
 (segment (start 145.82 107.68) (end 147.121142 106.378858) (width 0.2) (layer "F.Cu") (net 6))
 (segment (start 139.61 111.35) (end 142.98 111.35) (width 0.2) (layer "F.Cu") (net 6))
 (segment (start 138.36 116.97) (end 139 117.61) (width 0.2) (layer "F.Cu") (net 6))
 (segment (start 139.61 111.35) (end 138.36 112.6) (width 0.2) (layer "F.Cu") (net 6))
 (segment (start 139 117.61) (end 143.9203 117.61) (width 0.2) (layer "F.Cu") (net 6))
 (segment (start 138.36 112.6) (end 138.36 116.97) (width 0.2) (layer "F.Cu") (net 6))
 (segment (start 143.9203 117.61) (end 144.6 116.9303) (width 0.2) (layer "F.Cu") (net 6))
 (segment (start 144.6 116.9303) (end 144.6 116.03) (width 0.2) (layer "F.Cu") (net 6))
 (segment (start 143.19 85.165) (end 145.965 82.39) (width 0.2) (layer "B.Cu") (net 6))
 (segment (start 143.19 107.78) (end 143.19 85.165) (width 0.2) (layer "B.Cu") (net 6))
 (segment (start 147.18 102.861) (end 145.811 104.23) (width 0.2) (layer "B.Cu") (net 6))
 (segment (start 148.88 100.26) (end 147.18 101.96) (width 0.2) (layer "B.Cu") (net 6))
 (segment (start 139.62 111.35) (end 143.19 107.78) (width 0.2) (layer "B.Cu") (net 6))
 (segment (start 139.61 111.35) (end 139.62 111.35) (width 0.2) (layer "B.Cu") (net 6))
 (segment (start 147.18 101.96) (end 147.18 102.861) (width 0.2) (layer "B.Cu") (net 6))
 (segment (start 145.811 104.23) (end 143.19 104.23) (width 0.2) (layer "B.Cu") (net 6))
 (segment (start 149.5 99.92) (end 149.5 99.93) (width 0.2) (layer "B.Cu") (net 6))
 (segment (start 148.18 101.6779) (end 148.18 101.66) (width 0.2) (layer "F.Cu") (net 4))
 (segment (start 147.7575 102.9847) (end 147.3154 102.5425) (width 0.2) (layer "F.Cu") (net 4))
 (segment (start 147.3154 102.5425) (end 148.18 101.6779) (width 0.2) (layer "F.Cu") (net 4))
 (via (at 148.18 101.66) (size 0.5) (drill 0.3) (layers "F.Cu" "B.Cu") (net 4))
 (segment (start 148.18 101.66) (end 148.18 102.86) (width 0.2) (layer "B.Cu") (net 4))
 (segment (start 145.945 105.095) (end 145.945 123.29) (width 0.2) (layer "B.Cu") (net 4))
 (segment (start 148.18 102.86) (end 145.945 105.095) (width 0.2) (layer "B.Cu") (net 4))
 (segment (start 157.23 103.57) (end 151.2028 103.57) (width 0.2) (layer "F.Cu") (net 13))
 (segment (start 151.2028 103.57) (end 150.5153 104.2575) (width 0.2) (layer "F.Cu") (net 13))
 (segment (start 157.39 103.73) (end 157.23 103.57) (width 0.2) (layer "F.Cu") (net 13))
 (segment (start 153.6 104.08) (end 155.79 106.27) (width 0.2) (layer "F.Cu") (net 12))
 (segment (start 155.79 106.27) (end 157.39 106.27) (width 0.2) (layer "F.Cu") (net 12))
 (segment (start 151.329188 104.08) (end 153.6 104.08) (width 0.2) (layer "F.Cu") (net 12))
 (segment (start 150.833452 104.575736) (end 151.329188 104.08) (width 0.2) (layer "F.Cu") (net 12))
 (segment (start 157.39 108.81) (end 154.2192 108.81) (width 0.2) (layer "F.Cu") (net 11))
 (segment (start 154.2192 108.81) (end 150.8335 105.4243) (width 0.2) (layer "F.Cu") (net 11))
 (segment (start 157.39 116.43) (end 156.97 116.43) (width 0.2) (layer "F.Cu") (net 8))
 (segment (start 149.7 107.4728) (end 149.2425 107.0153) (width 0.2) (layer "F.Cu") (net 8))
 (segment (start 156.97 116.43) (end 149.7 109.16) (width 0.2) (layer "F.Cu") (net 8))
 (segment (start 149.7 109.16) (end 149.7 107.4728) (width 0.2) (layer "F.Cu") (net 8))
 (segment (start 157.39 118.52) (end 149.3664 110.4964) (width 0.2) (layer "F.Cu") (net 7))
 (segment (start 149.3664 107.7757) (end 149.3665 107.7756) (width 0.2) (layer "F.Cu") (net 7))
 (segment (start 149.3665 107.7756) (end 148.9243 107.3335) (width 0.2) (layer "F.Cu") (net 7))
 (segment (start 149.3664 110.4964) (end 149.3664 107.7757) (width 0.2) (layer "F.Cu") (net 7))
 (segment (start 157.39 118.97) (end 157.39 118.52) (width 0.2) (layer "F.Cu") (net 7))
 (segment (start 139.61 118.97) (end 144.91 118.97) (width 0.2) (layer "F.Cu") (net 29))
 (segment (start 147.6336 107.7756) (end 148.0757 107.3335) (width 0.2) (layer "F.Cu") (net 29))
 (segment (start 144.91 118.97) (end 147.6336 116.2464) (width 0.2) (layer "F.Cu") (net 29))
 (segment (start 147.6336 116.2464) (end 147.6336 107.7756) (width 0.2) (layer "F.Cu") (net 29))
 (segment (start 147.06 108.98) (end 147.06 107.7128) (width 0.2) (layer "F.Cu") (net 28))
 (segment (start 139.61 116.43) (end 147.06 108.98) (width 0.2) (layer "F.Cu") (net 28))
 (segment (start 147.06 107.7128) (end 147.7575 107.0153) (width 0.2) (layer "F.Cu") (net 28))
 (segment (start 141.41 113.89) (end 146.49 108.81) (width 0.2) (layer "F.Cu") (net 27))
 (segment (start 146.49 108.81) (end 146.49 107.646396) (width 0.2) (layer "F.Cu") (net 27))
 (segment (start 139.61 113.89) (end 141.41 113.89) (width 0.2) (layer "F.Cu") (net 27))
 (segment (start 146.49 107.646396) (end 147.43934 106.697056) (width 0.2) (layer "F.Cu") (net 27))
 (segment (start 146.9972 100.9472) (end 146.9972 102.8607) (width 0.2) (layer "F.Cu") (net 20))
 (segment (start 139.61 93.57) (end 139.62 93.57) (width 0.2) (layer "F.Cu") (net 20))
 (segment (start 139.62 93.57) (end 146.9972 100.9472) (width 0.2) (layer "F.Cu") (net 20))
 (segment (start 146.9972 102.8607) (end 147.4393 103.3029) (width 0.2) (layer "F.Cu") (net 20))
 (segment (start 144.0536 108.81) (end 146.8029 106.0607) (width 0.2) (layer "F.Cu") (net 26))
 (segment (start 139.61 108.81) (end 144.0536 108.81) (width 0.2) (layer "F.Cu") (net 26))
 (segment (start 139.63 106.29) (end 145.9372 106.29) (width 0.2) (layer "F.Cu") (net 25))
 (segment (start 145.9372 106.29) (end 146.4847 105.7425) (width 0.2) (layer "F.Cu") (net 25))
 (segment (start 139.61 106.27) (end 139.63 106.29) (width 0.2) (layer "F.Cu") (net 25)))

